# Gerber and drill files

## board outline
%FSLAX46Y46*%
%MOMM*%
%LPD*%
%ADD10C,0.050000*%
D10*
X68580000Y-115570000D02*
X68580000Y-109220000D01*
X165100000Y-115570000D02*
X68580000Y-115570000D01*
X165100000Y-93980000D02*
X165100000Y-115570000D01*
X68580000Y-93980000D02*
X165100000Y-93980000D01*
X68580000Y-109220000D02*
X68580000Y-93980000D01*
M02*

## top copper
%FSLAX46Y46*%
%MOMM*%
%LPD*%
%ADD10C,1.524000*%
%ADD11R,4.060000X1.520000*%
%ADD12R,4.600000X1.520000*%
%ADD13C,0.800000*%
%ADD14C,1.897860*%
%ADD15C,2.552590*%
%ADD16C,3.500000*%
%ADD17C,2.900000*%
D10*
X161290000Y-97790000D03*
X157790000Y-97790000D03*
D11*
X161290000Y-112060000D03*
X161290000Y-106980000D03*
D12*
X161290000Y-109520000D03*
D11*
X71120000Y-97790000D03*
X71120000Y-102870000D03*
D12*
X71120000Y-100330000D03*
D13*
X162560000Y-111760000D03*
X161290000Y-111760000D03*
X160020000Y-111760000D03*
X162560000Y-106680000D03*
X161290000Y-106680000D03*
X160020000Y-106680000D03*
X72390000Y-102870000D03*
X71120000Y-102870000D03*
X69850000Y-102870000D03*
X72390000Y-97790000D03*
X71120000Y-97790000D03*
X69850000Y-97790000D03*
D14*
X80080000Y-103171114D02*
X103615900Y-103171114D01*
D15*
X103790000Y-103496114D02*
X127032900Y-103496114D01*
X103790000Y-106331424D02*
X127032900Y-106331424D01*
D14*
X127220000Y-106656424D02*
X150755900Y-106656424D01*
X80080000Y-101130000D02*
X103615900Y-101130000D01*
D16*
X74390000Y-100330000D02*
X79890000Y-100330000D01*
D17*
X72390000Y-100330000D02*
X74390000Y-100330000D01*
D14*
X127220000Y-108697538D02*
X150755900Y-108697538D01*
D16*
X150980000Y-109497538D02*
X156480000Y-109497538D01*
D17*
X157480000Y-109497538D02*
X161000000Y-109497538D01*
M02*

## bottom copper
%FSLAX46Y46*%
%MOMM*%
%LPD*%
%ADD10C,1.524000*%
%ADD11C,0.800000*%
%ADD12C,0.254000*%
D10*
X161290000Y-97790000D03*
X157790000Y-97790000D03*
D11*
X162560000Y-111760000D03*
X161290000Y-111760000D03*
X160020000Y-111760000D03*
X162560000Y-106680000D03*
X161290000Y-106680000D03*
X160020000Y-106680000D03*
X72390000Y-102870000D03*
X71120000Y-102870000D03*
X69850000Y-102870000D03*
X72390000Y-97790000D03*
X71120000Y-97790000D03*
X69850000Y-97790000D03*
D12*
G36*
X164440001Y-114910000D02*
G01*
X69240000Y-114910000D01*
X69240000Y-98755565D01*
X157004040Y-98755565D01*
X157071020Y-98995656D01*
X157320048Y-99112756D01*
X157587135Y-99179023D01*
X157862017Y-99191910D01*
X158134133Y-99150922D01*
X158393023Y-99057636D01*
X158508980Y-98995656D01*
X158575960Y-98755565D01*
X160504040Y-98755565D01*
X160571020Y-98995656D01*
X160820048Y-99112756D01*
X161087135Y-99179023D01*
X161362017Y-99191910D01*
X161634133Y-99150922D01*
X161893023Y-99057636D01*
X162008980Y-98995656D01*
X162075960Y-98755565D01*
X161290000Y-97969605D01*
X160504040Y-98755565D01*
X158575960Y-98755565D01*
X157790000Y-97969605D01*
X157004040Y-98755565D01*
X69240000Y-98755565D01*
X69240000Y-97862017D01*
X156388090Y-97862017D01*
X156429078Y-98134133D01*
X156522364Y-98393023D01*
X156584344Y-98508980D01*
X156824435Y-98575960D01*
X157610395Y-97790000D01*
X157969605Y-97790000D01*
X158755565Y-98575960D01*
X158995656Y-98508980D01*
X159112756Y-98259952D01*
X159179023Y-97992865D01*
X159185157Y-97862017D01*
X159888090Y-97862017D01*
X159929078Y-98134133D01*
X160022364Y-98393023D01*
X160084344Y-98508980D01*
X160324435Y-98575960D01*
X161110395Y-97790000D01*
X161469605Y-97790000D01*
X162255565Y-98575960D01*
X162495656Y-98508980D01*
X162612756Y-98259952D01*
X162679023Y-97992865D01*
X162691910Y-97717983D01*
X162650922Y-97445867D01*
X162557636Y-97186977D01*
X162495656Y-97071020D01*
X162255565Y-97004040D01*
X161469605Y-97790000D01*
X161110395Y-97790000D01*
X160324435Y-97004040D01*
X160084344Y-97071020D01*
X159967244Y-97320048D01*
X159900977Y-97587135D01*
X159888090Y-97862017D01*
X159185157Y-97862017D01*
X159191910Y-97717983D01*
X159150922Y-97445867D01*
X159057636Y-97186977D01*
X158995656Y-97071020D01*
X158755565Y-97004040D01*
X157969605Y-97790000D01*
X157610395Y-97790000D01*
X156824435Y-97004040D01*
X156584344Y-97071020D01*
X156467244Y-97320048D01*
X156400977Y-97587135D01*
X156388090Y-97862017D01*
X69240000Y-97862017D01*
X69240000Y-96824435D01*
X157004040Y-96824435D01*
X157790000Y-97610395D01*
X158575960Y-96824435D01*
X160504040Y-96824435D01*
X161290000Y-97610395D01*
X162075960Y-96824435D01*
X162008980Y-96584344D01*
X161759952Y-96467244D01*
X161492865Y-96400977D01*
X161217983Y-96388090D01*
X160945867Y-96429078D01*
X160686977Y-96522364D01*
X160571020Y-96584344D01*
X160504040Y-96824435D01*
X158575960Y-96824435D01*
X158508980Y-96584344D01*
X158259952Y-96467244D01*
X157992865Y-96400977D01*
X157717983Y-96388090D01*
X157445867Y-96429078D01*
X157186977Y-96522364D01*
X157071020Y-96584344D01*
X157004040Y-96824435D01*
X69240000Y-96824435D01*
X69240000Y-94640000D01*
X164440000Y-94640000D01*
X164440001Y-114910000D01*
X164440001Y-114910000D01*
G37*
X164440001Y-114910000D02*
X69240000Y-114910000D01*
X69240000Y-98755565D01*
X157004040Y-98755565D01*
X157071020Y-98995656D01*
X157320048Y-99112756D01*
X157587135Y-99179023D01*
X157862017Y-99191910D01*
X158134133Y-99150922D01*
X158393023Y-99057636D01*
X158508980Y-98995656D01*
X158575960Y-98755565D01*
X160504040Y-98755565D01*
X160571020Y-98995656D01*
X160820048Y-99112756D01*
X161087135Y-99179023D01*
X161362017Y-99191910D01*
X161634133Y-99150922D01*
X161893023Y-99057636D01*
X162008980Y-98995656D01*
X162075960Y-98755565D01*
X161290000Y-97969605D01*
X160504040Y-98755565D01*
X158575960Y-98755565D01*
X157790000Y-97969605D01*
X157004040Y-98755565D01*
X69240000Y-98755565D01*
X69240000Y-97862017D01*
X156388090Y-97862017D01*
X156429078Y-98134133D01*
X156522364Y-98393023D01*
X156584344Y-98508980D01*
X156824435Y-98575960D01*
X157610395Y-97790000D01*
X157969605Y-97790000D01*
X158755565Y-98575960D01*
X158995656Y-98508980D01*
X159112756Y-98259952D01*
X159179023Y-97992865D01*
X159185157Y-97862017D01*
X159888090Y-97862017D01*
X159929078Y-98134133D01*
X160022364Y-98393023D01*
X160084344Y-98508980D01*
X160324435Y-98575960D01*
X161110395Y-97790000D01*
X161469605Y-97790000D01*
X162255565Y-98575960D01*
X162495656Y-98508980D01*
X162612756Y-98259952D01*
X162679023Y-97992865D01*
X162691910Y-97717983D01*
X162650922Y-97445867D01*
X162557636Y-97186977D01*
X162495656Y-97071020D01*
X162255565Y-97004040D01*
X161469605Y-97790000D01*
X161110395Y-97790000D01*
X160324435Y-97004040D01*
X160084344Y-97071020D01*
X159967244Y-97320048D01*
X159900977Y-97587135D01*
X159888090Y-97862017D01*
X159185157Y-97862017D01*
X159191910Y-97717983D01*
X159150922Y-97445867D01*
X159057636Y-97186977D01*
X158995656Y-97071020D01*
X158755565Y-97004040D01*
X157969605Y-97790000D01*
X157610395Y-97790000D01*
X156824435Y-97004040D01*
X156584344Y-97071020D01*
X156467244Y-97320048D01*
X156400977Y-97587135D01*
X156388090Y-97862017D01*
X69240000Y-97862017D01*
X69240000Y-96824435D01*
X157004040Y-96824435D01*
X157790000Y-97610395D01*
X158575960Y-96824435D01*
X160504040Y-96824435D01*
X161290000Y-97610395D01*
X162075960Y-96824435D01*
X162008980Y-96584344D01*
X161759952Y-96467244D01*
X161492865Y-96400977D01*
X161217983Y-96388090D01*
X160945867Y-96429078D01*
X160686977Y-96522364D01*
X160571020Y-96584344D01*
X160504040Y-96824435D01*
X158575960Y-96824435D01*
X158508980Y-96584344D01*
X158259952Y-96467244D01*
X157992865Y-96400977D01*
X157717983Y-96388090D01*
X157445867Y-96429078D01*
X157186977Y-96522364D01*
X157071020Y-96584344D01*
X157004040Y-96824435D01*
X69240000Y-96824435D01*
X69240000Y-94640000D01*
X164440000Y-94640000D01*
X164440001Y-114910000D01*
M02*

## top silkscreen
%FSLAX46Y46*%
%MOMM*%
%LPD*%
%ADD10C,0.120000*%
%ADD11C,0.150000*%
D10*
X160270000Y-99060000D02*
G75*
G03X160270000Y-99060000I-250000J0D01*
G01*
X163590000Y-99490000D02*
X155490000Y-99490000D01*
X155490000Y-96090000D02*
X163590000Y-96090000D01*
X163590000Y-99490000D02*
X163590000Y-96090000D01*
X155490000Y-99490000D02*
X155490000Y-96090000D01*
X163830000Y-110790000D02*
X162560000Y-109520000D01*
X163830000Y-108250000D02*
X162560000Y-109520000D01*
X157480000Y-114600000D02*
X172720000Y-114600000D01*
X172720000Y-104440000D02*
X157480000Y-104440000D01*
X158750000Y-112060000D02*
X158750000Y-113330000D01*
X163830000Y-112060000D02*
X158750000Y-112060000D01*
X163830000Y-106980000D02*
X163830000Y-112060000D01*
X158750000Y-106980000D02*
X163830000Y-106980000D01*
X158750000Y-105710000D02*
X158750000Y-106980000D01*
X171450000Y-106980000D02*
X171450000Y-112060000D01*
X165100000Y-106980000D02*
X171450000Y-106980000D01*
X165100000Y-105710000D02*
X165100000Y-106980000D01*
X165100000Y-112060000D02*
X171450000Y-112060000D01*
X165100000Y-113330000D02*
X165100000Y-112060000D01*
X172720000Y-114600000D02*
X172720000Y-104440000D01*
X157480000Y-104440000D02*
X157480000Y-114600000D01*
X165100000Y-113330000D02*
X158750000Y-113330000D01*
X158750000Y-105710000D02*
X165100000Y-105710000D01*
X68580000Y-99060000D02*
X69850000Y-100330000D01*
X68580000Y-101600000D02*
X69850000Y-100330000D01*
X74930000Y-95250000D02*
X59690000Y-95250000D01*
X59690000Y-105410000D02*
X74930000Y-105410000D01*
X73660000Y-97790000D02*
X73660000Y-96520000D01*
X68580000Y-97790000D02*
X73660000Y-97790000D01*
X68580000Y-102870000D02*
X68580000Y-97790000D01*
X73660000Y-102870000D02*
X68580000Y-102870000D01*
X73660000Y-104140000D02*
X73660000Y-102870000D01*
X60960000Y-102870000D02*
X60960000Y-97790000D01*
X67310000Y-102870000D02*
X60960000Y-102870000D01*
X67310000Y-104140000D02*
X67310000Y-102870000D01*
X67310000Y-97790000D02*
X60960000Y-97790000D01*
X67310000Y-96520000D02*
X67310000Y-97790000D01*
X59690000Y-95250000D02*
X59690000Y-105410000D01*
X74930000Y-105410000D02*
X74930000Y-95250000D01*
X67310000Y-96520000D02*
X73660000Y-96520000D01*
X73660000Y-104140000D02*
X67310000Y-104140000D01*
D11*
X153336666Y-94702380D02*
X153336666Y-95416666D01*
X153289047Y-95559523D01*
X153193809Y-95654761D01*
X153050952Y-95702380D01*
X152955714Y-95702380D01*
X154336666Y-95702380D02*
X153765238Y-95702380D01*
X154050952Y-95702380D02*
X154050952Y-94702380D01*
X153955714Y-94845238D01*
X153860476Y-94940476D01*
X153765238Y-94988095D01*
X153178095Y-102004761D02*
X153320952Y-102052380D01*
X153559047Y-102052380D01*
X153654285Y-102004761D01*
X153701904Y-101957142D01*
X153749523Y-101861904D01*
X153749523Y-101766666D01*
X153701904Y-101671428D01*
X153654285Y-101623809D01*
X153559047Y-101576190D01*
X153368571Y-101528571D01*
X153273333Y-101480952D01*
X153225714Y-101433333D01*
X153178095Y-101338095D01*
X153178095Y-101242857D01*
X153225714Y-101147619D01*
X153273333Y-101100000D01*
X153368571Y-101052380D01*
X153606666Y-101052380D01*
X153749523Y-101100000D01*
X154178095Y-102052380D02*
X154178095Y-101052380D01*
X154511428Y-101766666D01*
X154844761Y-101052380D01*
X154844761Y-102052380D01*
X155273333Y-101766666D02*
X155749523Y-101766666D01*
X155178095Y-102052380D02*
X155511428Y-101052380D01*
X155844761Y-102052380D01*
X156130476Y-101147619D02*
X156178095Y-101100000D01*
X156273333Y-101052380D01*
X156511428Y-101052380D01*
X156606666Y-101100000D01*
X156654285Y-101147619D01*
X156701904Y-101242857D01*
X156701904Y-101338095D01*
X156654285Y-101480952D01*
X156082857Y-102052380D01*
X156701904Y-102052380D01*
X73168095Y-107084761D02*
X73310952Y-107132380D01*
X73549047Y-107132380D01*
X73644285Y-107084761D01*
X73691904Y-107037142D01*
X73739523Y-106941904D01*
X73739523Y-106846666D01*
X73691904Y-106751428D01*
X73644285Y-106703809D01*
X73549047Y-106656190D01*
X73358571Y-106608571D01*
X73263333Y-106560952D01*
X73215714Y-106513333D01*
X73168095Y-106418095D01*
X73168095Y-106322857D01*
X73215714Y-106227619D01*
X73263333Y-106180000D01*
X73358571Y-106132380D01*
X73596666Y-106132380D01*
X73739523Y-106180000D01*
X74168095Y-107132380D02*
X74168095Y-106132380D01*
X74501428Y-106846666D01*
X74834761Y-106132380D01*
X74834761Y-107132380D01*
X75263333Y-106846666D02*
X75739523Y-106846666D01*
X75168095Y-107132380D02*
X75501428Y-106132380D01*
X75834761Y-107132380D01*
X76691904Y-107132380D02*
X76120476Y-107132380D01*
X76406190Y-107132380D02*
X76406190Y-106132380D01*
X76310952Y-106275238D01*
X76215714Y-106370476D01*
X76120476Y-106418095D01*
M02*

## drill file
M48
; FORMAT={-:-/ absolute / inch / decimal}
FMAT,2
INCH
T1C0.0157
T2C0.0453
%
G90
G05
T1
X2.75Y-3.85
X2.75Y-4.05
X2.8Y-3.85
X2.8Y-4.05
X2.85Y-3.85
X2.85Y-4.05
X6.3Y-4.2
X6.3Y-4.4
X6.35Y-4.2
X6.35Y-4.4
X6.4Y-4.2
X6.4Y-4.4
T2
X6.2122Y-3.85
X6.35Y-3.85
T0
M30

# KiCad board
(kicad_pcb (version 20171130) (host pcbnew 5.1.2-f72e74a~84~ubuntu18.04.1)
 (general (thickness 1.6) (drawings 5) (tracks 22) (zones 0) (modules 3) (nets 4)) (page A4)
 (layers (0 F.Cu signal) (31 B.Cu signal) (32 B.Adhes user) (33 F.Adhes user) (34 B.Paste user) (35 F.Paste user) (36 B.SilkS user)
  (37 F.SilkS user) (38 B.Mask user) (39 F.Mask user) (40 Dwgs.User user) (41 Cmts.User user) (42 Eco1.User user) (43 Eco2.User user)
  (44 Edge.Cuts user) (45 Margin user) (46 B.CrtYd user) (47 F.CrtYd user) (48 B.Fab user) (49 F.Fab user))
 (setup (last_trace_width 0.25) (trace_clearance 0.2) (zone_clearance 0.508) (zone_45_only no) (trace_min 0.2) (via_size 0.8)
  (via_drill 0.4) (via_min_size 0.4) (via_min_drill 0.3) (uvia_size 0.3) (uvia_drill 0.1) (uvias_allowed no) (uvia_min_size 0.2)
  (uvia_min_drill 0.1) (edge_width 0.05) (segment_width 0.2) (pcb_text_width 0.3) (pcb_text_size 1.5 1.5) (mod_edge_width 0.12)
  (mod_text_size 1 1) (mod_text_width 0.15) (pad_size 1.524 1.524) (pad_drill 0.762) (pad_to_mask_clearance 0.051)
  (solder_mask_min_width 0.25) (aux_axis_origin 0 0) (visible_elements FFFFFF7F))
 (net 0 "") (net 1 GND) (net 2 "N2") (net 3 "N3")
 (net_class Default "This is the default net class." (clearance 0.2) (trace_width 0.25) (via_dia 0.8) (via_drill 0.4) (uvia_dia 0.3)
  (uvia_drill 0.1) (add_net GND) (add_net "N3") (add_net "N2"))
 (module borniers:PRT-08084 (layer F.Cu) (at 161.29 102.87)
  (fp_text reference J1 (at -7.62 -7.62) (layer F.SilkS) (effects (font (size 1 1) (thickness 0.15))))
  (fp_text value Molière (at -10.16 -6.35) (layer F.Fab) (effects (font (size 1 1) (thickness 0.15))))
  (fp_circle (center -1.27 -3.81) (end -1.02 -3.81) (layer F.SilkS) (width 0.12))
  (fp_line (start 2.3 -3.38) (end -5.8 -3.38) (layer F.SilkS) (width 0.12))
  (fp_line (start -5.8 -6.78) (end 2.3 -6.78) (layer F.SilkS) (width 0.12))
  (fp_line (start 2.3 -3.38) (end 2.3 -6.78) (layer F.SilkS) (width 0.12))
  (fp_line (start -5.8 -3.38) (end -5.8 -6.78) (layer F.SilkS) (width 0.12))
  (pad 2 thru_hole circle (at 0 -5.08) (size 1.524 1.524) (drill 1.15) (layers *.Cu *.Mask) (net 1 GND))
  (pad 1 thru_hole circle (at -3.5 -5.08) (size 1.524 1.524) (drill 1.15) (layers *.Cu *.Mask) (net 1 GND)))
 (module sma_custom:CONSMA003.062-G (layer F.Cu) (at 165.1 112.06)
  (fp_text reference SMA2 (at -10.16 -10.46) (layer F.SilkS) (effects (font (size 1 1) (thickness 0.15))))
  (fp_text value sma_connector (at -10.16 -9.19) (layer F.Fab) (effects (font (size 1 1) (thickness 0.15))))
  (fp_line (start -1.27 -1.27) (end -2.54 -2.54) (layer F.SilkS) (width 0.12))
  (fp_line (start -1.27 -3.81) (end -2.54 -2.54) (layer F.SilkS) (width 0.12))
  (fp_line (start -7.62 2.54) (end 7.62 2.54) (layer F.SilkS) (width 0.12))
  (fp_line (start 7.62 -7.62) (end -7.62 -7.62) (layer F.SilkS) (width 0.12))
  (fp_line (start -6.35 0) (end -6.35 1.27) (layer F.SilkS) (width 0.12))
  (fp_line (start -1.27 0) (end -6.35 0) (layer F.SilkS) (width 0.12))
  (fp_line (start -1.27 -5.08) (end -1.27 0) (layer F.SilkS) (width 0.12))
  (fp_line (start -6.35 -5.08) (end -1.27 -5.08) (layer F.SilkS) (width 0.12))
  (fp_line (start -6.35 -6.35) (end -6.35 -5.08) (layer F.SilkS) (width 0.12))
  (fp_line (start 6.35 -5.08) (end 6.35 0) (layer F.SilkS) (width 0.12))
  (fp_line (start 0 -5.08) (end 6.35 -5.08) (layer F.SilkS) (width 0.12))
  (fp_line (start 0 -6.35) (end 0 -5.08) (layer F.SilkS) (width 0.12))
  (fp_line (start 0 0) (end 6.35 0) (layer F.SilkS) (width 0.12))
  (fp_line (start 0 1.27) (end 0 0) (layer F.SilkS) (width 0.12))
  (fp_line (start 7.62 2.54) (end 7.62 -7.62) (layer F.SilkS) (width 0.12))
  (fp_line (start -7.62 -7.62) (end -7.62 2.54) (layer F.SilkS) (width 0.12))
  (fp_line (start 0 1.27) (end -6.35 1.27) (layer F.SilkS) (width 0.12))
  (fp_line (start -6.35 -6.35) (end 0 -6.35) (layer F.SilkS) (width 0.12))
  (pad 3 smd rect (at -3.81 0) (size 4.06 1.52) (layers F.Cu F.Paste F.Mask) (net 1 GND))
  (pad 2 smd rect (at -3.81 -5.08) (size 4.06 1.52) (layers F.Cu F.Paste F.Mask) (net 1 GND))
  (pad 1 smd rect (at -3.81 -2.54) (size 4.6 1.52) (layers F.Cu F.Paste F.Mask) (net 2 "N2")))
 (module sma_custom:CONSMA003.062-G (layer F.Cu) (at 67.31 97.79 180)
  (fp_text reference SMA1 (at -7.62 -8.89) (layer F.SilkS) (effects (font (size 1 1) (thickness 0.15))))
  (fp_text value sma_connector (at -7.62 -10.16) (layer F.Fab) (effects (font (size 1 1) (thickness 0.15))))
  (fp_line (start -1.27 -1.27) (end -2.54 -2.54) (layer F.SilkS) (width 0.12))
  (fp_line (start -1.27 -3.81) (end -2.54 -2.54) (layer F.SilkS) (width 0.12))
  (fp_line (start -7.62 2.54) (end 7.62 2.54) (layer F.SilkS) (width 0.12))
  (fp_line (start 7.62 -7.62) (end -7.62 -7.62) (layer F.SilkS) (width 0.12))
  (fp_line (start -6.35 0) (end -6.35 1.27) (layer F.SilkS) (width 0.12))
  (fp_line (start -1.27 0) (end -6.35 0) (layer F.SilkS) (width 0.12))
  (fp_line (start -1.27 -5.08) (end -1.27 0) (layer F.SilkS) (width 0.12))
  (fp_line (start -6.35 -5.08) (end -1.27 -5.08) (layer F.SilkS) (width 0.12))
  (fp_line (start -6.35 -6.35) (end -6.35 -5.08) (layer F.SilkS) (width 0.12))
  (fp_line (start 6.35 -5.08) (end 6.35 0) (layer F.SilkS) (width 0.12))
  (fp_line (start 0 -5.08) (end 6.35 -5.08) (layer F.SilkS) (width 0.12))
  (fp_line (start 0 -6.35) (end 0 -5.08) (layer F.SilkS) (width 0.12))
  (fp_line (start 0 0) (end 6.35 0) (layer F.SilkS) (width 0.12))
  (fp_line (start 0 1.27) (end 0 0) (layer F.SilkS) (width 0.12))
  (fp_line (start 7.62 2.54) (end 7.62 -7.62) (layer F.SilkS) (width 0.12))
  (fp_line (start -7.62 -7.62) (end -7.62 2.54) (layer F.SilkS) (width 0.12))
  (fp_line (start 0 1.27) (end -6.35 1.27) (layer F.SilkS) (width 0.12))
  (fp_line (start -6.35 -6.35) (end 0 -6.35) (layer F.SilkS) (width 0.12))
  (pad 3 smd rect (at -3.81 0 180) (size 4.06 1.52) (layers F.Cu F.Paste F.Mask) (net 1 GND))
  (pad 2 smd rect (at -3.81 -5.08 180) (size 4.06 1.52) (layers F.Cu F.Paste F.Mask) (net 1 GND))
  (pad 1 smd rect (at -3.81 -2.54 180) (size 4.6 1.52) (layers F.Cu F.Paste F.Mask) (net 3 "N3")))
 (gr_line (start 68.58 115.57) (end 68.58 109.22) (layer Edge.Cuts) (width 0.05))
 (gr_line (start 165.1 115.57) (end 68.58 115.57) (layer Edge.Cuts) (width 0.05))
 (gr_line (start 165.1 93.98) (end 165.1 115.57) (layer Edge.Cuts) (width 0.05))
 (gr_line (start 68.58 93.98) (end 165.1 93.98) (layer Edge.Cuts) (width 0.05))
 (gr_line (start 68.58 109.22) (end 68.58 93.98) (layer Edge.Cuts) (width 0.05))
 (segment (start 80.08 103.171114) (end 103.6159 103.171114) (width 1.89786) (layer F.Cu) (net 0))
 (segment (start 103.79 103.496114) (end 127.0329 103.496114) (width 2.55259) (layer F.Cu) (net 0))
 (segment (start 103.79 106.331424) (end 127.0329 106.331424) (width 2.55259) (layer F.Cu) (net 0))
 (segment (start 127.22 106.656424) (end 150.7559 106.656424) (width 1.89786) (layer F.Cu) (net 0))
 (via (at 162.56 111.76) (size 0.8) (drill 0.4) (layers F.Cu B.Cu) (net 1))
 (via (at 161.29 111.76) (size 0.8) (drill 0.4) (layers F.Cu B.Cu) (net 1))
 (via (at 160.02 111.76) (size 0.8) (drill 0.4) (layers F.Cu B.Cu) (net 1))
 (via (at 162.56 106.68) (size 0.8) (drill 0.4) (layers F.Cu B.Cu) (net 1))
 (via (at 161.29 106.68) (size 0.8) (drill 0.4) (layers F.Cu B.Cu) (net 1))
 (via (at 160.02 106.68) (size 0.8) (drill 0.4) (layers F.Cu B.Cu) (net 1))
 (via (at 72.39 102.87) (size 0.8) (drill 0.4) (layers F.Cu B.Cu) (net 1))
 (via (at 71.12 102.87) (size 0.8) (drill 0.4) (layers F.Cu B.Cu) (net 1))
 (via (at 69.85 102.87) (size 0.8) (drill 0.4) (layers F.Cu B.Cu) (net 1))
 (via (at 72.39 97.79) (size 0.8) (drill 0.4) (layers F.Cu B.Cu) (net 1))
 (via (at 71.12 97.79) (size 0.8) (drill 0.4) (layers F.Cu B.Cu) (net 1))
 (via (at 69.85 97.79) (size 0.8) (drill 0.4) (layers F.Cu B.Cu) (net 1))
 (segment (start 80.08 101.13) (end 103.6159 101.13) (width 1.89786) (layer F.Cu) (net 3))
 (segment (start 74.39 100.33) (end 79.89 100.33) (width 3.5) (layer F.Cu) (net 3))
 (segment (start 72.39 100.33) (end 74.39 100.33) (width 2.9) (layer F.Cu) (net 3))
 (segment (start 127.22 108.697538) (end 150.7559 108.697538) (width 1.89786) (layer F.Cu) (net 2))
 (segment (start 150.98 109.497538) (end 156.48 109.497538) (width 3.5) (layer F.Cu) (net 2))
 (segment (start 157.48 109.497538) (end 161 109.497538) (width 2.9) (layer F.Cu) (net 2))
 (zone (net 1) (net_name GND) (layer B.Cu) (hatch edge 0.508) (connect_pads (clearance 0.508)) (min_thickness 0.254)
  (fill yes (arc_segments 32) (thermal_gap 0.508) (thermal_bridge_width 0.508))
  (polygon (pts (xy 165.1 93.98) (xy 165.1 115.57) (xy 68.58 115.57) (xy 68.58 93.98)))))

